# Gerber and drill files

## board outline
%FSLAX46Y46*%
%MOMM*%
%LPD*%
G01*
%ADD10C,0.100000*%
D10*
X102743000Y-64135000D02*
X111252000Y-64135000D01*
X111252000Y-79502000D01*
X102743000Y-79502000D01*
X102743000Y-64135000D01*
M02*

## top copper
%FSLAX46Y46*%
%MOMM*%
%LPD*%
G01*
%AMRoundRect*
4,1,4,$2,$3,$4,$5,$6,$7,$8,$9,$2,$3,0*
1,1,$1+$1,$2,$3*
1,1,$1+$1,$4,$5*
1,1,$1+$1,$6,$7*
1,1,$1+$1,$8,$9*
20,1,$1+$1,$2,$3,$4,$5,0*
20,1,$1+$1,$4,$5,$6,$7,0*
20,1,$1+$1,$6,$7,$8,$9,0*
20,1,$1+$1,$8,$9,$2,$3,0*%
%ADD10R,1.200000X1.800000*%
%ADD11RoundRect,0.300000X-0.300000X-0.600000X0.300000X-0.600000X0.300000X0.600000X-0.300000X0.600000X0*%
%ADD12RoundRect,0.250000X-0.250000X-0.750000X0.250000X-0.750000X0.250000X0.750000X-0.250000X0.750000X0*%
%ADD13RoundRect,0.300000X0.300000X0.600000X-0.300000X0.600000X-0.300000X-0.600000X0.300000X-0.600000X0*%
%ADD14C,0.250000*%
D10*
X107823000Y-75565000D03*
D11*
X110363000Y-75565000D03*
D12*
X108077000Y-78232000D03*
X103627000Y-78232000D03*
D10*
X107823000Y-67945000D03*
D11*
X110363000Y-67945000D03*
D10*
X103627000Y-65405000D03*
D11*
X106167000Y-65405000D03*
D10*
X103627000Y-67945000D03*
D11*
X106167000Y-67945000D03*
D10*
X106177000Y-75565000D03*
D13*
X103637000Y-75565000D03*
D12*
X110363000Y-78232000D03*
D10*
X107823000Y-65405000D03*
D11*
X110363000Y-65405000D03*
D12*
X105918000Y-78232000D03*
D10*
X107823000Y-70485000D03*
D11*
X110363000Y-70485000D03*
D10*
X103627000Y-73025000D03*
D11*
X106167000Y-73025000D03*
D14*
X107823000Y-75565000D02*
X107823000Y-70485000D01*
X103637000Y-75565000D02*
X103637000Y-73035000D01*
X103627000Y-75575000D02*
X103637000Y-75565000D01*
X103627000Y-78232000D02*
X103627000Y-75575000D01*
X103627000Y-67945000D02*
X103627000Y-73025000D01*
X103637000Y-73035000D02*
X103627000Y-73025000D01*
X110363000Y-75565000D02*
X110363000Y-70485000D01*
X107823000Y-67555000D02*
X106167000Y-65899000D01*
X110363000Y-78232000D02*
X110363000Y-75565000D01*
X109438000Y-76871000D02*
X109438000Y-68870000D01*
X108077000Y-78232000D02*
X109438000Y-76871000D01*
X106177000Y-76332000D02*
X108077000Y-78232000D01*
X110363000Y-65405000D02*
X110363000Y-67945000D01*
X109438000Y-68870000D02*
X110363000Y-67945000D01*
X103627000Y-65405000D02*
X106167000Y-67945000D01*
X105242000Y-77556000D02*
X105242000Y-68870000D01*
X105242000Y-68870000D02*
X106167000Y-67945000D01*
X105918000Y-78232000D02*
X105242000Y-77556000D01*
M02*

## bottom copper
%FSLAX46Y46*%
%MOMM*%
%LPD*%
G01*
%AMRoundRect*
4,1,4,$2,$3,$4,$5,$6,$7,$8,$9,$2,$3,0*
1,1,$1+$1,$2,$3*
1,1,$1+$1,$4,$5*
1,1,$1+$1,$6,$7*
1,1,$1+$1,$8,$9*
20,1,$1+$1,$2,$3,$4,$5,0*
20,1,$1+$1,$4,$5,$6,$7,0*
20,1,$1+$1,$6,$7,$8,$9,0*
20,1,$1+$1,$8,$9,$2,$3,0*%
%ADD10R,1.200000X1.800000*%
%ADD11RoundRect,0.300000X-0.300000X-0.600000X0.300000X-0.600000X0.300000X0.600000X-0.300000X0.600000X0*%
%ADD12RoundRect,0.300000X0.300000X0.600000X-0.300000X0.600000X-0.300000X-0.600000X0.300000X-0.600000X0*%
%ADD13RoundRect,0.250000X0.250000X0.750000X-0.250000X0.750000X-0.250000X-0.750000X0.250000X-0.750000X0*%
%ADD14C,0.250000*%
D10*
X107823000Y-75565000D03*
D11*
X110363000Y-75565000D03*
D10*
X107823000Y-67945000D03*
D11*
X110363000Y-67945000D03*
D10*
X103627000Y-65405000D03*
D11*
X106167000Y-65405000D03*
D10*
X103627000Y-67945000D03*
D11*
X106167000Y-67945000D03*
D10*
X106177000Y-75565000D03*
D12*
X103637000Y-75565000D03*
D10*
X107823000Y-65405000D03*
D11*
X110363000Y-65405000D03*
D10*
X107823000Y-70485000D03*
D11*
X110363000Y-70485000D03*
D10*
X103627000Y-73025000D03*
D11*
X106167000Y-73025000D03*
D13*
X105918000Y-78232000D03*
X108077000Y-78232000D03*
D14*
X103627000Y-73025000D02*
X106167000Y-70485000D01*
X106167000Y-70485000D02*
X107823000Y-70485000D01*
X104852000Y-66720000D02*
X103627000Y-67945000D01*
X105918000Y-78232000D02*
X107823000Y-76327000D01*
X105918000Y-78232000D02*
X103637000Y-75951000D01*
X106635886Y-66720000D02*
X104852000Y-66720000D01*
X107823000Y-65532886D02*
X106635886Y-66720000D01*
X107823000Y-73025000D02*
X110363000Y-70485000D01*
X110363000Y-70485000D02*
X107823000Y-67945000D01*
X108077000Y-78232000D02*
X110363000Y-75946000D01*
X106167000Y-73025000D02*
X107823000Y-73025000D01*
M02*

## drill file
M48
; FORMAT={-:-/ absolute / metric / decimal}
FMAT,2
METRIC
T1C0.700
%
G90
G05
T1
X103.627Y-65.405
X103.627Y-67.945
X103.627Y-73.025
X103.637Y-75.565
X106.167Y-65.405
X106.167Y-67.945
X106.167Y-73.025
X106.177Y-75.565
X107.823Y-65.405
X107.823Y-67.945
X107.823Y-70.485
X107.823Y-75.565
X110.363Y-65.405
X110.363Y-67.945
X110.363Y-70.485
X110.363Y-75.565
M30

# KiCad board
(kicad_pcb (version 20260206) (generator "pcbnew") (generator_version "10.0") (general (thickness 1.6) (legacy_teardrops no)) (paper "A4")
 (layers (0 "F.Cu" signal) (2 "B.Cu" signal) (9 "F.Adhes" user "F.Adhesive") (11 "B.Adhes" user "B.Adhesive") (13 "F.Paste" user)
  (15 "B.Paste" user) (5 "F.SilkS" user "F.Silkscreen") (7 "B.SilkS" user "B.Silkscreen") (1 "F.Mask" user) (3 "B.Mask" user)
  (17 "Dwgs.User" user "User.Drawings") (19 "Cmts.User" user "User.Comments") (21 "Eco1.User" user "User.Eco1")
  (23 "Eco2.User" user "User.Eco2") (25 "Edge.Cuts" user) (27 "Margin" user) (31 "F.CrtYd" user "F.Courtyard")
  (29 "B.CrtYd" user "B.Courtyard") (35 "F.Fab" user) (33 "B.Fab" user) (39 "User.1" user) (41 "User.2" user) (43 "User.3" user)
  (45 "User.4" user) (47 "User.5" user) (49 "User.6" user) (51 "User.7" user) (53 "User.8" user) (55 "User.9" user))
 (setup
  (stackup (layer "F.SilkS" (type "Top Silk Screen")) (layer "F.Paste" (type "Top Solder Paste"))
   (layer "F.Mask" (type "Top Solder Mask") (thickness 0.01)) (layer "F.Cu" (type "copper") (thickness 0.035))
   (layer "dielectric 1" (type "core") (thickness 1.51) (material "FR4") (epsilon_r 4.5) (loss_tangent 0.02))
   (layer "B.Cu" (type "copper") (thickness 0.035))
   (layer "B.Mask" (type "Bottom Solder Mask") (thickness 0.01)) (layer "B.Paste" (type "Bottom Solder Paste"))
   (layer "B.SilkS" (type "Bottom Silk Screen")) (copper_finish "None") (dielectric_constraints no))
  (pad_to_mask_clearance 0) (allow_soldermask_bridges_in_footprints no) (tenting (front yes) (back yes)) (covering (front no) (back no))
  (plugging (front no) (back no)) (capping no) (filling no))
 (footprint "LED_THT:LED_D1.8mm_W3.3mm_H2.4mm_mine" (layer "F.Cu") (at 107.823 75.565)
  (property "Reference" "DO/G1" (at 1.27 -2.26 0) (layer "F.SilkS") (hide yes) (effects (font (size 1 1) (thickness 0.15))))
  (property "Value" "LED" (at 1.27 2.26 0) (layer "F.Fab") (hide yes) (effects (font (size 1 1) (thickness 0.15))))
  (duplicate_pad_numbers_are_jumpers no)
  (pad "1" thru_hole rect (at 0 0) (size 1.2 1.8) (drill 0.7) (layers "*.Cu" "*.Mask") (remove_unused_layers no) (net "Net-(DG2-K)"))
  (pad "2" thru_hole roundrect (at 2.54 0) (size 1.2 1.8) (drill 0.7) (layers "*.Cu" "*.Mask") (remove_unused_layers no)
   (roundrect_rratio 0.25) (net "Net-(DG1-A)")))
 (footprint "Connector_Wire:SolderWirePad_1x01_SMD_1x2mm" (layer "F.Cu") (at 108.077 78.232)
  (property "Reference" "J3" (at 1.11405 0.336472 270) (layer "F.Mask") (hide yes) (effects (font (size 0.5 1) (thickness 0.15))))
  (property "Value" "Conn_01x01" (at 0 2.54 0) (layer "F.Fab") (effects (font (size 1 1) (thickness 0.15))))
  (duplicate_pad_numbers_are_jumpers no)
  (pad "1" smd roundrect (at 0 0) (size 1 2) (layers "F.Cu" "F.Mask" "F.Paste") (roundrect_rratio 0.25) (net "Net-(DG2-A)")))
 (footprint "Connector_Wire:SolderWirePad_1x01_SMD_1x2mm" (layer "F.Cu") (at 103.627 78.232)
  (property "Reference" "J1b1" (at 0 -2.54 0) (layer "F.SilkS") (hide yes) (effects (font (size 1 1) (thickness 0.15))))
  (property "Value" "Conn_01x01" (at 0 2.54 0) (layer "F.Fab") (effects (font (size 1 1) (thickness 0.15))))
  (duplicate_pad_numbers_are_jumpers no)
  (pad "1" smd roundrect (at 0 0) (size 1 2) (layers "F.Cu" "F.Mask" "F.Paste") (roundrect_rratio 0.25) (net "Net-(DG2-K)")))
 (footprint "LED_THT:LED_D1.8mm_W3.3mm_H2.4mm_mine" (layer "F.Cu") (at 107.823 67.945)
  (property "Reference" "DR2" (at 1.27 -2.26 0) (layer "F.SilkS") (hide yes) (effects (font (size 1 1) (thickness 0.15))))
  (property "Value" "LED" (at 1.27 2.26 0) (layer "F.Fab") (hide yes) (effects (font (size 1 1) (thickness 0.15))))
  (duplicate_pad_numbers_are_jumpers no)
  (pad "1" thru_hole rect (at 0 0) (size 1.2 1.8) (drill 0.7) (layers "*.Cu" "*.Mask") (remove_unused_layers no) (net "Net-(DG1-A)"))
  (pad "2" thru_hole roundrect (at 2.54 0) (size 1.2 1.8) (drill 0.7) (layers "*.Cu" "*.Mask") (remove_unused_layers no)
   (roundrect_rratio 0.25) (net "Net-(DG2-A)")))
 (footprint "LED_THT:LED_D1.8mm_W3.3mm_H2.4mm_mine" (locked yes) (layer "F.Cu") (at 103.627 65.405)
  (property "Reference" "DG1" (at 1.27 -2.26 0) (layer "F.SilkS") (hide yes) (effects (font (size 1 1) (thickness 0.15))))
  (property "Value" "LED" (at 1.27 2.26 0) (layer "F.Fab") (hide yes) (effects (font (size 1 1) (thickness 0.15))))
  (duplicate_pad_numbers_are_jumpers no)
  (pad "1" thru_hole rect (at 0 0) (size 1.2 1.8) (drill 0.7) (layers "*.Cu" "*.Mask") (remove_unused_layers no) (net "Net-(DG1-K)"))
  (pad "2" thru_hole roundrect (at 2.54 0) (size 1.2 1.8) (drill 0.7) (layers "*.Cu" "*.Mask") (remove_unused_layers no)
   (roundrect_rratio 0.25) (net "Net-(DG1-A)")))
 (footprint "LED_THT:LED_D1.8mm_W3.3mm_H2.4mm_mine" (layer "F.Cu") (at 103.627 67.945)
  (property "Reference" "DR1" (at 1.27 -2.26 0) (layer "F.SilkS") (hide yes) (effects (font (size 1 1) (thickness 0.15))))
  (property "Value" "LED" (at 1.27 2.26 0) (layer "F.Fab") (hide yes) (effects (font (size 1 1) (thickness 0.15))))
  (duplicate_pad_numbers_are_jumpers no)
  (pad "1" thru_hole rect (at 0 0) (size 1.2 1.8) (drill 0.7) (layers "*.Cu" "*.Mask") (remove_unused_layers no) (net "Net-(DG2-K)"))
  (pad "2" thru_hole roundrect (at 2.54 0) (size 1.2 1.8) (drill 0.7) (layers "*.Cu" "*.Mask") (remove_unused_layers no)
   (roundrect_rratio 0.25) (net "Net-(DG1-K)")))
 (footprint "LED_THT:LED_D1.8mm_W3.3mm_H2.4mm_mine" (layer "F.Cu") (at 106.177 75.565 180)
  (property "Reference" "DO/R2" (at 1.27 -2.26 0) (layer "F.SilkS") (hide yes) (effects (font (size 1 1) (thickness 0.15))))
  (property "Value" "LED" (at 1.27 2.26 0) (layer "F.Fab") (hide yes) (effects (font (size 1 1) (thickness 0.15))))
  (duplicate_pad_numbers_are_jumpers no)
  (pad "1" thru_hole rect (at 0 0 180) (size 1.2 1.8) (drill 0.7) (layers "*.Cu" "*.Mask") (remove_unused_layers no) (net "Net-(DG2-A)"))
  (pad "2" thru_hole roundrect (at 2.54 0 180) (size 1.2 1.8) (drill 0.7) (layers "*.Cu" "*.Mask") (remove_unused_layers no)
   (roundrect_rratio 0.25) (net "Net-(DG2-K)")))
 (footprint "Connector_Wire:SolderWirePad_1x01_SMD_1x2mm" (layer "F.Cu") (at 110.363 78.232)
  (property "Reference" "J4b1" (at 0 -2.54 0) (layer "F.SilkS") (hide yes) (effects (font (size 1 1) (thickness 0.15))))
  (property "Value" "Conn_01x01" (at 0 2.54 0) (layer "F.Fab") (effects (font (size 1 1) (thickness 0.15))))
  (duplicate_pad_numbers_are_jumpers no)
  (pad "1" smd roundrect (at 0 0) (size 1 2) (layers "F.Cu" "F.Mask" "F.Paste") (roundrect_rratio 0.25) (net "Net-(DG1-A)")))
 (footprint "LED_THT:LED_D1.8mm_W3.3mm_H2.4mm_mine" (layer "F.Cu") (at 107.823 65.405)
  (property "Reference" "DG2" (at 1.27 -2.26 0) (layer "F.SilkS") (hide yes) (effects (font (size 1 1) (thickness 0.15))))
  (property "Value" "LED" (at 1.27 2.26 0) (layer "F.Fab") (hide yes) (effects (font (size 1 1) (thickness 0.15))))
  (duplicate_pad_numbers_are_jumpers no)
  (pad "1" thru_hole rect (at 0 0) (size 1.2 1.8) (drill 0.7) (layers "*.Cu" "*.Mask") (remove_unused_layers no) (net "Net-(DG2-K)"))
  (pad "2" thru_hole roundrect (at 2.54 0) (size 1.2 1.8) (drill 0.7) (layers "*.Cu" "*.Mask") (remove_unused_layers no)
   (roundrect_rratio 0.25) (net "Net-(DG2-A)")))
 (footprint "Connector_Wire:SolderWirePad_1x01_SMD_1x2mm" (layer "F.Cu") (at 105.918 78.232)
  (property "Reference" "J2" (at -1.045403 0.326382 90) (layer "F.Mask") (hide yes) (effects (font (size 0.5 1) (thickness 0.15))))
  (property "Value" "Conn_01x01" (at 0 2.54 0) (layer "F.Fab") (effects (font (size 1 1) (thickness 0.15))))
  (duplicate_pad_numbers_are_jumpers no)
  (pad "1" smd roundrect (at 0 0) (size 1 2) (layers "F.Cu" "F.Mask" "F.Paste") (roundrect_rratio 0.25) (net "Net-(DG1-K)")))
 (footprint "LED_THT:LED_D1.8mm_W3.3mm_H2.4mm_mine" (layer "F.Cu") (at 107.823 70.485)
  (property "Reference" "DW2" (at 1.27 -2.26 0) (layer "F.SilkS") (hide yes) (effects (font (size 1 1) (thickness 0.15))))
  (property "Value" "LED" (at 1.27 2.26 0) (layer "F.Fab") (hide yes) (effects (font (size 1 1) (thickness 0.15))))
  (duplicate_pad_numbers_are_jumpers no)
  (pad "1" thru_hole rect (at 0 0) (size 1.2 1.8) (drill 0.7) (layers "*.Cu" "*.Mask") (remove_unused_layers no) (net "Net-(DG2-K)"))
  (pad "2" thru_hole roundrect (at 2.54 0) (size 1.2 1.8) (drill 0.7) (layers "*.Cu" "*.Mask") (remove_unused_layers no)
   (roundrect_rratio 0.25) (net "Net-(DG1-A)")))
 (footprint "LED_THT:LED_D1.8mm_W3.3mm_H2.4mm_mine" (layer "F.Cu") (at 103.627 73.025)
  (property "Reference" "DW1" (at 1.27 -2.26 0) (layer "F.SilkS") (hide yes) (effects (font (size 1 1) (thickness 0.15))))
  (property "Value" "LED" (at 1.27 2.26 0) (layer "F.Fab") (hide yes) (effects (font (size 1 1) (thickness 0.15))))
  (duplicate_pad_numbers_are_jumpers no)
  (pad "1" thru_hole rect (at 0 0) (size 1.2 1.8) (drill 0.7) (layers "*.Cu" "*.Mask") (remove_unused_layers no) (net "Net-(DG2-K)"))
  (pad "2" thru_hole roundrect (at 2.54 0) (size 1.2 1.8) (drill 0.7) (layers "*.Cu" "*.Mask") (remove_unused_layers no)
   (roundrect_rratio 0.25) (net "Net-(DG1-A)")))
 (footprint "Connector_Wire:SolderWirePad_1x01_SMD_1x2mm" (layer "B.Cu") (at 105.918 78.232 180)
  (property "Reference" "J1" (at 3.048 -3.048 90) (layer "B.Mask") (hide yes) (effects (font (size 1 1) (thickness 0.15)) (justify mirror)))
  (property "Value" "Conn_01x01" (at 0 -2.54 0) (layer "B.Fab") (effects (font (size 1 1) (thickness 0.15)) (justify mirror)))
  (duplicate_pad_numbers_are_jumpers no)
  (pad "1" smd roundrect (at 0 0 180) (size 1 2) (layers "B.Cu" "B.Mask" "B.Paste") (roundrect_rratio 0.25) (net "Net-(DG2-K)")))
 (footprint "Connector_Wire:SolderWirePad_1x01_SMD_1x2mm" (layer "B.Cu") (at 108.077 78.232 180)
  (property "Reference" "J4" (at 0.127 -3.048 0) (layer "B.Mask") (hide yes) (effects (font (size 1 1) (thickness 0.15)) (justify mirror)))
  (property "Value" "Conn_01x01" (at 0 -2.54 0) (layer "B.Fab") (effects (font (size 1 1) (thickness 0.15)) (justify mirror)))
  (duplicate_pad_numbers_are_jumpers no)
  (pad "1" smd roundrect (at 0 0 180) (size 1 2) (layers "B.Cu" "B.Mask" "B.Paste") (roundrect_rratio 0.25) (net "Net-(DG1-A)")))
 (gr_rect (start 102.743 64.135) (end 111.252 79.502) (stroke (width 0.1) (type default)) (fill no) (layer "Edge.Cuts"))
 (segment (start 107.823 75.565) (end 107.823 70.485) (width 0.25) (layer "F.Cu") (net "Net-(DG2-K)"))
 (segment (start 103.637 75.565) (end 103.637 73.035) (width 0.25) (layer "F.Cu") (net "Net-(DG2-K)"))
 (segment (start 103.627 75.575) (end 103.637 75.565) (width 0.25) (layer "F.Cu") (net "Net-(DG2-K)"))
 (segment (start 103.627 78.232) (end 103.627 75.575) (width 0.25) (layer "F.Cu") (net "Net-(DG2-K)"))
 (segment (start 103.627 67.945) (end 103.627 73.025) (width 0.25) (layer "F.Cu") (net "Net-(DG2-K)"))
 (segment (start 103.637 73.035) (end 103.627 73.025) (width 0.25) (layer "F.Cu") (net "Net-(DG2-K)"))
 (segment (start 103.627 73.025) (end 106.167 70.485) (width 0.25) (layer "B.Cu") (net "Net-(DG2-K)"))
 (segment (start 106.167 70.485) (end 107.823 70.485) (width 0.25) (layer "B.Cu") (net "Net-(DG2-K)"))
 (segment (start 104.852 66.72) (end 103.627 67.945) (width 0.25) (layer "B.Cu") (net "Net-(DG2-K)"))
 (segment (start 105.918 78.232) (end 107.823 76.327) (width 0.25) (layer "B.Cu") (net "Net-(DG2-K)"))
 (segment (start 105.918 78.232) (end 103.637 75.951) (width 0.25) (layer "B.Cu") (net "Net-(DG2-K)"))
 (segment (start 106.635886 66.72) (end 104.852 66.72) (width 0.25) (layer "B.Cu") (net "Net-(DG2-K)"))
 (segment (start 107.823 65.532886) (end 106.635886 66.72) (width 0.25) (layer "B.Cu") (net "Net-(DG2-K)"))
 (segment (start 110.363 75.565) (end 110.363 70.485) (width 0.25) (layer "F.Cu") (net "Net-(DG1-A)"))
 (segment (start 107.823 67.555) (end 106.167 65.899) (width 0.25) (layer "F.Cu") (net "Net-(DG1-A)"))
 (segment (start 110.363 78.232) (end 110.363 75.565) (width 0.25) (layer "F.Cu") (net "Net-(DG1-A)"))
 (segment (start 107.823 73.025) (end 110.363 70.485) (width 0.25) (layer "B.Cu") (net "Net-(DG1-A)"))
 (segment (start 110.363 70.485) (end 107.823 67.945) (width 0.25) (layer "B.Cu") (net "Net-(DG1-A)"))
 (segment (start 108.077 78.232) (end 110.363 75.946) (width 0.25) (layer "B.Cu") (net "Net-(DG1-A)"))
 (segment (start 106.167 73.025) (end 107.823 73.025) (width 0.25) (layer "B.Cu") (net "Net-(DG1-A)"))
 (segment (start 109.438 76.871) (end 109.438 68.87) (width 0.25) (layer "F.Cu") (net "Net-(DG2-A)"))
 (segment (start 108.077 78.232) (end 109.438 76.871) (width 0.25) (layer "F.Cu") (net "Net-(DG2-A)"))
 (segment (start 106.177 76.332) (end 108.077 78.232) (width 0.25) (layer "F.Cu") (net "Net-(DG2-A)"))
 (segment (start 110.363 65.405) (end 110.363 67.945) (width 0.25) (layer "F.Cu") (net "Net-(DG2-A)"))
 (segment (start 109.438 68.87) (end 110.363 67.945) (width 0.25) (layer "F.Cu") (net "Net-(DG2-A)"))
 (segment (start 103.627 65.405) (end 106.167 67.945) (width 0.25) (layer "F.Cu") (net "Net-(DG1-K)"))
 (segment (start 105.242 77.556) (end 105.242 68.87) (width 0.25) (layer "F.Cu") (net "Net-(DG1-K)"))
 (segment (start 105.242 68.87) (end 106.167 67.945) (width 0.25) (layer "F.Cu") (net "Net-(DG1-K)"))
 (segment (start 105.918 78.232) (end 105.242 77.556) (width 0.25) (layer "F.Cu") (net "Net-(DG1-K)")))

